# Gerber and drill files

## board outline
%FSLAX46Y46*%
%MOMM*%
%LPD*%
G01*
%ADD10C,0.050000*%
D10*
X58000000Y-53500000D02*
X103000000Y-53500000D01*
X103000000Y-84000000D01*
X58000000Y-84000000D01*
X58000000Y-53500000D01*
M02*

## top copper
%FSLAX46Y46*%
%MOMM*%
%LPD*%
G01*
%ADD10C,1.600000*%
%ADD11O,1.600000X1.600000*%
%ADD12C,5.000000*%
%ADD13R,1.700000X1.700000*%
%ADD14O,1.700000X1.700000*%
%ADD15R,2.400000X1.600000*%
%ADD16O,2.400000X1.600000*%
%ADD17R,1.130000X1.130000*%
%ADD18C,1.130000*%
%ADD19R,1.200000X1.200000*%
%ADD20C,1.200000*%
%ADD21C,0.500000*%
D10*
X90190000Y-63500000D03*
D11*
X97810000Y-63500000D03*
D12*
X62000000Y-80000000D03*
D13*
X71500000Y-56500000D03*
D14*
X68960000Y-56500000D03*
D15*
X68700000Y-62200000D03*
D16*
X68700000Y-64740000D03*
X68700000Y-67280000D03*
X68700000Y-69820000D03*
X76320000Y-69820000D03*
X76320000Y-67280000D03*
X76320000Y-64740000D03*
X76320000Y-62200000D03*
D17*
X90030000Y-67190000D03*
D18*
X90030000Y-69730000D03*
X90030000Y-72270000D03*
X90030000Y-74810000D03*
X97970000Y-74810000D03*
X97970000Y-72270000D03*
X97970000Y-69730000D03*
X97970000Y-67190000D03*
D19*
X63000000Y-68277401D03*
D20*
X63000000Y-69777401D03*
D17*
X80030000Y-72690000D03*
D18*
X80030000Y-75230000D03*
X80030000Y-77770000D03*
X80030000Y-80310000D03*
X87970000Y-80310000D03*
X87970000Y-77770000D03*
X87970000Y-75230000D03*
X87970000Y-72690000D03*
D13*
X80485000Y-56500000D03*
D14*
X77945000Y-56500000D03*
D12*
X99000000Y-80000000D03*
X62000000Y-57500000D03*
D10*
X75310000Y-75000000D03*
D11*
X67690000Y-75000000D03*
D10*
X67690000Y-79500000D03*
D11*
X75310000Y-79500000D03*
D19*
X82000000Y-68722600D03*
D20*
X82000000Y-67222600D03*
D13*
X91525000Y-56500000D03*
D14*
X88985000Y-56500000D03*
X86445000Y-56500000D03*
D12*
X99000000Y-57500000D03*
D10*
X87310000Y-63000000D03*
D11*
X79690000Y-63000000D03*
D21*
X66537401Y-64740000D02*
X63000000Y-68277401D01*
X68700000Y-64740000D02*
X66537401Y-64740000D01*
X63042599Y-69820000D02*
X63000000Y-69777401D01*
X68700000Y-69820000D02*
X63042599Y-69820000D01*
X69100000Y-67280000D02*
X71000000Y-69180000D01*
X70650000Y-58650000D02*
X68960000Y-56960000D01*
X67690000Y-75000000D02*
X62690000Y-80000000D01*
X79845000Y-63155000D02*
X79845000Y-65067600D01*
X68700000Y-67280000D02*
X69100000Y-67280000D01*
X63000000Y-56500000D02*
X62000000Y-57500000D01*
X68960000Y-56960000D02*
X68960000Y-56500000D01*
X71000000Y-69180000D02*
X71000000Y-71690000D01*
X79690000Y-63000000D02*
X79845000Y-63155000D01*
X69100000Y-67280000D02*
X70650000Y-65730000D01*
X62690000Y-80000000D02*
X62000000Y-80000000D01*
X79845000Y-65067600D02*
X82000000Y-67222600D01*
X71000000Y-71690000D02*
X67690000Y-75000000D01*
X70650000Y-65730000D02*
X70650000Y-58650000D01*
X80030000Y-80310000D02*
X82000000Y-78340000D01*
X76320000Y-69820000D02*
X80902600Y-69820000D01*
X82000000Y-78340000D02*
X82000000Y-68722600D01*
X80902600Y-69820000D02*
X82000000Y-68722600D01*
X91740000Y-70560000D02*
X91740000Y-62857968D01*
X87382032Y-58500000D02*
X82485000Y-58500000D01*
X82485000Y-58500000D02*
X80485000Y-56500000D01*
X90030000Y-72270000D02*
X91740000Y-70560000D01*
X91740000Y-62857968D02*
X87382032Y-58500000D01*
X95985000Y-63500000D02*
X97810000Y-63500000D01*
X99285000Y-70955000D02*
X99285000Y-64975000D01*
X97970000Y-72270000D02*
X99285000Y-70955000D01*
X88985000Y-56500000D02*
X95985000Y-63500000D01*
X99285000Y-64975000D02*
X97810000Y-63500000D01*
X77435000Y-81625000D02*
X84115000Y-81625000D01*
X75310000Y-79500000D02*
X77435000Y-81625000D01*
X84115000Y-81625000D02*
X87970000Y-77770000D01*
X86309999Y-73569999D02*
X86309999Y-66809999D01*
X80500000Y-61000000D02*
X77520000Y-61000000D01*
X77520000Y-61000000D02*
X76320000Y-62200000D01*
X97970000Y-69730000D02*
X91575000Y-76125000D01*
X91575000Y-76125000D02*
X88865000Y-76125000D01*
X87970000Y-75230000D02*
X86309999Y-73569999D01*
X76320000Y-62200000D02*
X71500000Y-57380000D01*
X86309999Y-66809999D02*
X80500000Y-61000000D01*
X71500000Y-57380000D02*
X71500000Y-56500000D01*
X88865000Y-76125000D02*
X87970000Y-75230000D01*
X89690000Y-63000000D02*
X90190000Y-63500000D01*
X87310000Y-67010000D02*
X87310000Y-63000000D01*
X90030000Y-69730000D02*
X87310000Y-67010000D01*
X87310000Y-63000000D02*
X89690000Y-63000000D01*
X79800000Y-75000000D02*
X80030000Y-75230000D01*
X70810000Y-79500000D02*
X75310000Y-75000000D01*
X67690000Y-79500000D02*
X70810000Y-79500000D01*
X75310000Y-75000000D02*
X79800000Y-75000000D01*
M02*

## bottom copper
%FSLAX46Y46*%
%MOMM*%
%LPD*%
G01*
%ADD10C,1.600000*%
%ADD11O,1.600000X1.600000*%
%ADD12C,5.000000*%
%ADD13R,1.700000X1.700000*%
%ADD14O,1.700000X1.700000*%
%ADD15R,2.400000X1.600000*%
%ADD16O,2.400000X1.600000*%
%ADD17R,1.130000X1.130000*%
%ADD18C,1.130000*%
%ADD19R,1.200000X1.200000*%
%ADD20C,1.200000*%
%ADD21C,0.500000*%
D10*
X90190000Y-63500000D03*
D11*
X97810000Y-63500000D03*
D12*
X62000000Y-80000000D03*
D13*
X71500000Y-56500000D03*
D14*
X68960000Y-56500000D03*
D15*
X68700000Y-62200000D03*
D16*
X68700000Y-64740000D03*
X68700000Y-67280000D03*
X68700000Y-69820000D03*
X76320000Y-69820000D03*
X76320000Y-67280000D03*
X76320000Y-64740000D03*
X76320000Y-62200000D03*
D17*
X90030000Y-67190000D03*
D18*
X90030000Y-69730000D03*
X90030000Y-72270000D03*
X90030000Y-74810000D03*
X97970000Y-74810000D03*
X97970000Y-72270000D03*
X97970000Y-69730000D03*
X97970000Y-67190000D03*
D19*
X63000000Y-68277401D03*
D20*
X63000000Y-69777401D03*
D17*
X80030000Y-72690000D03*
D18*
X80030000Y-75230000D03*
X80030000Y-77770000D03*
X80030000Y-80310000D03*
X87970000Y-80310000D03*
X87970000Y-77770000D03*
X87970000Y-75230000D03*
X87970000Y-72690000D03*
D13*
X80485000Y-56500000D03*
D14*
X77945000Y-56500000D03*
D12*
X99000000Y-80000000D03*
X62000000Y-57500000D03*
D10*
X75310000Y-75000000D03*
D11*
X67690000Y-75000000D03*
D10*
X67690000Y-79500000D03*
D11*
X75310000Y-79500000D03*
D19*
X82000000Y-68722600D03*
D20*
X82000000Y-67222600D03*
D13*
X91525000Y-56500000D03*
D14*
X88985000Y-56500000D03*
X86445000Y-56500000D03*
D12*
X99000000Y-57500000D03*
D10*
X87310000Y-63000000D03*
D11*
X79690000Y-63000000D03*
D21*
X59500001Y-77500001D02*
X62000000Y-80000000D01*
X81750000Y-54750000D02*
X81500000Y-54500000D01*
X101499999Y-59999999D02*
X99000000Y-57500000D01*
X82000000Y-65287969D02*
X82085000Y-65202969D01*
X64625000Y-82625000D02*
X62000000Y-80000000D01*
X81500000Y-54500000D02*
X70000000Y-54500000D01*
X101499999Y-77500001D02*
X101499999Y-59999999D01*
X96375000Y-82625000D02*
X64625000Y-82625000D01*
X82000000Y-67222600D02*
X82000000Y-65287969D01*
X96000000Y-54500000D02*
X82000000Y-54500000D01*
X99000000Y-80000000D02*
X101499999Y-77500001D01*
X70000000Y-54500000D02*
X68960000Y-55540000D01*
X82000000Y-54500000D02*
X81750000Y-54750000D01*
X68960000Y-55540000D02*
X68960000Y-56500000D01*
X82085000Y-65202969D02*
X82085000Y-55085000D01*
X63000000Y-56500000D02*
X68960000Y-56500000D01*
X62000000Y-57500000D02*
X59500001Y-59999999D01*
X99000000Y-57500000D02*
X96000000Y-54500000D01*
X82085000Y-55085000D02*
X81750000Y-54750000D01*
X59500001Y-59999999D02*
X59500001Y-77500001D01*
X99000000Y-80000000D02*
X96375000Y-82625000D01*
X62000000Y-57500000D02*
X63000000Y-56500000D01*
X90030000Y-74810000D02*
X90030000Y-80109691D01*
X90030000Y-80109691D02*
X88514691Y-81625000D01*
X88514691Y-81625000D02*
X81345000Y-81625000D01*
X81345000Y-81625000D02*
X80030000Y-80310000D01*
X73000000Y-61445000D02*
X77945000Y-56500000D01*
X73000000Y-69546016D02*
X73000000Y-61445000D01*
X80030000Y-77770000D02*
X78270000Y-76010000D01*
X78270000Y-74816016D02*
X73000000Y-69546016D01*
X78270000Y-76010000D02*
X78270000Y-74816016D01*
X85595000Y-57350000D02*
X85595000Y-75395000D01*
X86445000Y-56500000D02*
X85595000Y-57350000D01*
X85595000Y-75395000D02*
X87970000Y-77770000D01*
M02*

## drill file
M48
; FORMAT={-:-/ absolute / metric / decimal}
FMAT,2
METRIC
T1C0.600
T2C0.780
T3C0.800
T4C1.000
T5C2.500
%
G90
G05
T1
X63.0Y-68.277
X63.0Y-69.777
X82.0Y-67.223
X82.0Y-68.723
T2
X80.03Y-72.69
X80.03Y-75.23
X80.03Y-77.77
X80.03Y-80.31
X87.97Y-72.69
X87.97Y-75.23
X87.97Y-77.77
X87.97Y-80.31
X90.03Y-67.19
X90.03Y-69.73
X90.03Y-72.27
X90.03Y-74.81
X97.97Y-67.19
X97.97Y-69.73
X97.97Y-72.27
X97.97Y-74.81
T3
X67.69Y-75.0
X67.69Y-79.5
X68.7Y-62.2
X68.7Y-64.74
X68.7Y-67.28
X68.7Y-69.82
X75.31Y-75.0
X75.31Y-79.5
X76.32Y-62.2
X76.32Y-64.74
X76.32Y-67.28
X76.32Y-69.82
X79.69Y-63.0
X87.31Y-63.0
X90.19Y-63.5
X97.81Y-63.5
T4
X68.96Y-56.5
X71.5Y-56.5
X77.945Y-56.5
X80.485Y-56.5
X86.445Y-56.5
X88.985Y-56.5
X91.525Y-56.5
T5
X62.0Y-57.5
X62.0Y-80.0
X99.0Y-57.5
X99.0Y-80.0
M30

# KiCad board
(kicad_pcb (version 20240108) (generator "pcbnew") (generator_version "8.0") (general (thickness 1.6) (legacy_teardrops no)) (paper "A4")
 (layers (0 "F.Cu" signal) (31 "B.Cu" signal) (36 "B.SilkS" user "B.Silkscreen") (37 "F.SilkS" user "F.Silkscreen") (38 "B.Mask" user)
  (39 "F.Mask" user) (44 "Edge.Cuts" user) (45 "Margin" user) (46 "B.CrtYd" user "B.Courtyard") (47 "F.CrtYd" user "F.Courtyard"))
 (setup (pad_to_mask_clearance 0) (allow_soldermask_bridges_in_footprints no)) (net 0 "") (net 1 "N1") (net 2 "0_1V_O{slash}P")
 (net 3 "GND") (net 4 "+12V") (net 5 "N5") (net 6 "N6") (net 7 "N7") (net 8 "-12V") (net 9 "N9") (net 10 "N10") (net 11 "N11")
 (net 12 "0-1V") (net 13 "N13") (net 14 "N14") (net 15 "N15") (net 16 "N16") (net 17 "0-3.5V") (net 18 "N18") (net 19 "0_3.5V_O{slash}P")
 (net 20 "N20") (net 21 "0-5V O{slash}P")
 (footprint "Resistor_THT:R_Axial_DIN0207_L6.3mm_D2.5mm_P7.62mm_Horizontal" (layer "F.Cu") (at 90.19 63.5)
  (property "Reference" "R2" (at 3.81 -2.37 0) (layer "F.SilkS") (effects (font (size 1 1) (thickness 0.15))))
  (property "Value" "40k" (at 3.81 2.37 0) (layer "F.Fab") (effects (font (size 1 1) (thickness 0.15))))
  (pad "1" thru_hole circle (at 0 0) (size 1.6 1.6) (drill 0.8) (layers "*.Cu" "*.Mask") (remove_unused_layers no) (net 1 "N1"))
  (pad "2" thru_hole oval (at 7.62 0) (size 1.6 1.6) (drill 0.8) (layers "*.Cu" "*.Mask") (remove_unused_layers no) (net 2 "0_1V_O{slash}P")))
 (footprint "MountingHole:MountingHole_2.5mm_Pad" (layer "F.Cu") (at 62 80 180)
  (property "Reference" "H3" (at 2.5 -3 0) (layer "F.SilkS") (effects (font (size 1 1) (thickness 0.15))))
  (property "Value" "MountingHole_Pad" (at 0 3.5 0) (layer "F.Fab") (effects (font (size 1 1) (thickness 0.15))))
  (pad "1" thru_hole circle (at 0 0 180) (size 5 5) (drill 2.5) (layers "*.Cu" "*.Mask") (remove_unused_layers no) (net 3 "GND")))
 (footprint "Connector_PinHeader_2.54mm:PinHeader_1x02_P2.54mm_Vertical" (layer "F.Cu") (at 71.5 56.5 -90)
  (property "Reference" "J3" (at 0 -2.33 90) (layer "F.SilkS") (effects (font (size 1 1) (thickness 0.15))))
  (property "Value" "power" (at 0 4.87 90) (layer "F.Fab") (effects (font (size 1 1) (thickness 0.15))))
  (pad "1" thru_hole rect (at 0 0 270) (size 1.7 1.7) (drill 1) (layers "*.Cu" "*.Mask") (remove_unused_layers no) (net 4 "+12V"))
  (pad "2" thru_hole oval (at 0 2.54 270) (size 1.7 1.7) (drill 1) (layers "*.Cu" "*.Mask") (remove_unused_layers no) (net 3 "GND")))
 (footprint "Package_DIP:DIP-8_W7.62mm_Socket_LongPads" (layer "F.Cu") (at 68.7 62.2)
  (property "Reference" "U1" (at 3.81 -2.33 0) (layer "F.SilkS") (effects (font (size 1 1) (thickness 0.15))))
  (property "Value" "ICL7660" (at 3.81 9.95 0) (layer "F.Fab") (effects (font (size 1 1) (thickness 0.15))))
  (pad "1" thru_hole rect (at 0 0) (size 2.4 1.6) (drill 0.8) (layers "*.Cu" "*.Mask") (remove_unused_layers no) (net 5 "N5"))
  (pad "2" thru_hole oval (at 0 2.54) (size 2.4 1.6) (drill 0.8) (layers "*.Cu" "*.Mask") (remove_unused_layers no) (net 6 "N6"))
  (pad "3" thru_hole oval (at 0 5.08) (size 2.4 1.6) (drill 0.8) (layers "*.Cu" "*.Mask") (remove_unused_layers no) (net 3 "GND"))
  (pad "4" thru_hole oval (at 0 7.62) (size 2.4 1.6) (drill 0.8) (layers "*.Cu" "*.Mask") (remove_unused_layers no) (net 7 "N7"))
  (pad "5" thru_hole oval (at 7.62 7.62) (size 2.4 1.6) (drill 0.8) (layers "*.Cu" "*.Mask") (remove_unused_layers no) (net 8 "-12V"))
  (pad "6" thru_hole oval (at 7.62 5.08) (size 2.4 1.6) (drill 0.8) (layers "*.Cu" "*.Mask") (remove_unused_layers no) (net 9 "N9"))
  (pad "7" thru_hole oval (at 7.62 2.54) (size 2.4 1.6) (drill 0.8) (layers "*.Cu" "*.Mask") (remove_unused_layers no) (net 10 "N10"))
  (pad "8" thru_hole oval (at 7.62 0) (size 2.4 1.6) (drill 0.8) (layers "*.Cu" "*.Mask") (remove_unused_layers no) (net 4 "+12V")))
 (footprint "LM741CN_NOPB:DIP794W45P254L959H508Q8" (layer "F.Cu") (at 94 71)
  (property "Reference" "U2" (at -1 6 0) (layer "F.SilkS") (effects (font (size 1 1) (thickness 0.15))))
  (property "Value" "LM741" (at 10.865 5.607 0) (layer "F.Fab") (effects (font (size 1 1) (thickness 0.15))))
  (pad "1" thru_hole rect (at -3.97 -3.81) (size 1.13 1.13) (drill 0.78) (layers "*.Cu" "*.Mask") (remove_unused_layers no) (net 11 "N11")
   (solder_mask_margin 0.102))
  (pad "2" thru_hole circle (at -3.97 -1.27) (size 1.13 1.13) (drill 0.78) (layers "*.Cu" "*.Mask") (remove_unused_layers no) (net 1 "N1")
   (solder_mask_margin 0.102))
  (pad "3" thru_hole circle (at -3.97 1.27) (size 1.13 1.13) (drill 0.78) (layers "*.Cu" "*.Mask") (remove_unused_layers no) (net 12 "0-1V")
   (solder_mask_margin 0.102))
  (pad "4" thru_hole circle (at -3.97 3.81) (size 1.13 1.13) (drill 0.78) (layers "*.Cu" "*.Mask") (remove_unused_layers no) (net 8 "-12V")
   (solder_mask_margin 0.102))
  (pad "5" thru_hole circle (at 3.97 3.81) (size 1.13 1.13) (drill 0.78) (layers "*.Cu" "*.Mask") (remove_unused_layers no) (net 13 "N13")
   (solder_mask_margin 0.102))
  (pad "6" thru_hole circle (at 3.97 1.27) (size 1.13 1.13) (drill 0.78) (layers "*.Cu" "*.Mask") (remove_unused_layers no)
   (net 2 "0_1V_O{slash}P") (solder_mask_margin 0.102))
  (pad "7" thru_hole circle (at 3.97 -1.27) (size 1.13 1.13) (drill 0.78) (layers "*.Cu" "*.Mask") (remove_unused_layers no) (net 4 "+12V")
   (solder_mask_margin 0.102))
  (pad "8" thru_hole circle (at 3.97 -3.81) (size 1.13 1.13) (drill 0.78) (layers "*.Cu" "*.Mask") (remove_unused_layers no) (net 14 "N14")
   (solder_mask_margin 0.102)))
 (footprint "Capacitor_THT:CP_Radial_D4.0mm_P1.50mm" (layer "F.Cu") (at 63 68.277401 -90)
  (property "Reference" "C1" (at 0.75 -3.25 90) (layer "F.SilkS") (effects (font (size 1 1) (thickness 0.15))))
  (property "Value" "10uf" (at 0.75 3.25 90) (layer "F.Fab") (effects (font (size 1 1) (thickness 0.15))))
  (pad "1" thru_hole rect (at 0 0 270) (size 1.2 1.2) (drill 0.6) (layers "*.Cu" "*.Mask") (remove_unused_layers no) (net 6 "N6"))
  (pad "2" thru_hole circle (at 1.5 0 270) (size 1.2 1.2) (drill 0.6) (layers "*.Cu" "*.Mask") (remove_unused_layers no) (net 7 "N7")))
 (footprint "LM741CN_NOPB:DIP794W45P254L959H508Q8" (layer "F.Cu") (at 84 76.5)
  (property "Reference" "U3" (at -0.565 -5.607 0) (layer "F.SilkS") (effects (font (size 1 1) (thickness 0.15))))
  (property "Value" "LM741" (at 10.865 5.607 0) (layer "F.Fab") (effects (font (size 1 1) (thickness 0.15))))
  (pad "1" thru_hole rect (at -3.97 -3.81) (size 1.13 1.13) (drill 0.78) (layers "*.Cu" "*.Mask") (remove_unused_layers no) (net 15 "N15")
   (solder_mask_margin 0.102))
  (pad "2" thru_hole circle (at -3.97 -1.27) (size 1.13 1.13) (drill 0.78) (layers "*.Cu" "*.Mask") (remove_unused_layers no) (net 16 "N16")
   (solder_mask_margin 0.102))
  (pad "3" thru_hole circle (at -3.97 1.27) (size 1.13 1.13) (drill 0.78) (layers "*.Cu" "*.Mask") (remove_unused_layers no)
   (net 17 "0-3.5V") (solder_mask_margin 0.102))
  (pad "4" thru_hole circle (at -3.97 3.81) (size 1.13 1.13) (drill 0.78) (layers "*.Cu" "*.Mask") (remove_unused_layers no) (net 8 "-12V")
   (solder_mask_margin 0.102))
  (pad "5" thru_hole circle (at 3.97 3.81) (size 1.13 1.13) (drill 0.78) (layers "*.Cu" "*.Mask") (remove_unused_layers no) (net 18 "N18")
   (solder_mask_margin 0.102))
  (pad "6" thru_hole circle (at 3.97 1.27) (size 1.13 1.13) (drill 0.78) (layers "*.Cu" "*.Mask") (remove_unused_layers no)
   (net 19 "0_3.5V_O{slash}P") (solder_mask_margin 0.102))
  (pad "7" thru_hole circle (at 3.97 -1.27) (size 1.13 1.13) (drill 0.78) (layers "*.Cu" "*.Mask") (remove_unused_layers no) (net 4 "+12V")
   (solder_mask_margin 0.102))
  (pad "8" thru_hole circle (at 3.97 -3.81) (size 1.13 1.13) (drill 0.78) (layers "*.Cu" "*.Mask") (remove_unused_layers no) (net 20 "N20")
   (solder_mask_margin 0.102)))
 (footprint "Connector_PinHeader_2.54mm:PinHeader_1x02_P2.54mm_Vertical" (layer "F.Cu") (at 80.485 56.5 -90)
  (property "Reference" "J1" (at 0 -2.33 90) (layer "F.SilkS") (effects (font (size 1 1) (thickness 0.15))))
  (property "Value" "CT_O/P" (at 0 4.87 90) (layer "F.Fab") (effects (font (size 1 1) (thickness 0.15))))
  (pad "1" thru_hole rect (at 0 0 270) (size 1.7 1.7) (drill 1) (layers "*.Cu" "*.Mask") (remove_unused_layers no) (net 12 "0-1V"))
  (pad "2" thru_hole oval (at 0 2.54 270) (size 1.7 1.7) (drill 1) (layers "*.Cu" "*.Mask") (remove_unused_layers no) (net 17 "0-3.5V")))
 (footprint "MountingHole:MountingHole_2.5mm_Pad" (layer "F.Cu") (at 99 80 180)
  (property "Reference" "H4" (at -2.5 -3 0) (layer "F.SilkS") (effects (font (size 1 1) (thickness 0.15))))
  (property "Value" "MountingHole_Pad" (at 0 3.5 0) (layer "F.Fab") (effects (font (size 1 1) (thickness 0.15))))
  (pad "1" thru_hole circle (at 0 0 180) (size 5 5) (drill 2.5) (layers "*.Cu" "*.Mask") (remove_unused_layers no) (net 3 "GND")))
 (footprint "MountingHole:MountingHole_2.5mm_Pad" (layer "F.Cu") (at 62 57.5 180)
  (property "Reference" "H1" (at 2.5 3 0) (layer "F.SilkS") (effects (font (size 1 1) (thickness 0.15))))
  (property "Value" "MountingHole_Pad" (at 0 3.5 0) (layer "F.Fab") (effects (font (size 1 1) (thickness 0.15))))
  (pad "1" thru_hole circle (at 0 0 180) (size 5 5) (drill 2.5) (layers "*.Cu" "*.Mask") (remove_unused_layers no) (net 3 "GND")))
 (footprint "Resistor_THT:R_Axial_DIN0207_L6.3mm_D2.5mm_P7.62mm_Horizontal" (layer "F.Cu") (at 75.31 75 180)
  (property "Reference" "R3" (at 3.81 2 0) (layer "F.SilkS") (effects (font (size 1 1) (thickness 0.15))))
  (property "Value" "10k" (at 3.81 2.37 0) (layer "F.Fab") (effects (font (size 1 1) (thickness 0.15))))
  (pad "1" thru_hole circle (at 0 0 180) (size 1.6 1.6) (drill 0.8) (layers "*.Cu" "*.Mask") (remove_unused_layers no) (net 16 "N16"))
  (pad "2" thru_hole oval (at 7.62 0 180) (size 1.6 1.6) (drill 0.8) (layers "*.Cu" "*.Mask") (remove_unused_layers no) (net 3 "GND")))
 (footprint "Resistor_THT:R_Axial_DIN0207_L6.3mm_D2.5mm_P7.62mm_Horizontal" (layer "F.Cu") (at 67.69 79.5)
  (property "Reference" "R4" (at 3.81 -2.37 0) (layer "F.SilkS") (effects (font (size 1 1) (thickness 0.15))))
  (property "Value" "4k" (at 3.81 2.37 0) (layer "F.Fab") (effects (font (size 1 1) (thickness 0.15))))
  (pad "1" thru_hole circle (at 0 0) (size 1.6 1.6) (drill 0.8) (layers "*.Cu" "*.Mask") (remove_unused_layers no) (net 16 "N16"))
  (pad "2" thru_hole oval (at 7.62 0) (size 1.6 1.6) (drill 0.8) (layers "*.Cu" "*.Mask") (remove_unused_layers no)
   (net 19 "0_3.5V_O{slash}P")))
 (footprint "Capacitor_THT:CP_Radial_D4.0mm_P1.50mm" (layer "F.Cu") (at 82 68.7226 90)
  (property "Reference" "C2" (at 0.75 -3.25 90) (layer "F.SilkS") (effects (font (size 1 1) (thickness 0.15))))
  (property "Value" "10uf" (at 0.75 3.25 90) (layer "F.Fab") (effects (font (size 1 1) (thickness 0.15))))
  (pad "1" thru_hole rect (at 0 0 90) (size 1.2 1.2) (drill 0.6) (layers "*.Cu" "*.Mask") (remove_unused_layers no) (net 8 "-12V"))
  (pad "2" thru_hole circle (at 1.5 0 90) (size 1.2 1.2) (drill 0.6) (layers "*.Cu" "*.Mask") (remove_unused_layers no) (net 3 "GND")))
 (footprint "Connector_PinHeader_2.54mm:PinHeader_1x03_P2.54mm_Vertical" (layer "F.Cu") (at 91.525 56.5 -90)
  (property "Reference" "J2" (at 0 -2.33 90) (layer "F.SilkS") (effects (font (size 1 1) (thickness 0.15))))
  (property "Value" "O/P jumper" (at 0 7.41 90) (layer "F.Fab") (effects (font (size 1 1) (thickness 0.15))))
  (pad "1" thru_hole rect (at 0 0 270) (size 1.7 1.7) (drill 1) (layers "*.Cu" "*.Mask") (remove_unused_layers no) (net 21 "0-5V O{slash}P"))
  (pad "2" thru_hole oval (at 0 2.54 270) (size 1.7 1.7) (drill 1) (layers "*.Cu" "*.Mask") (remove_unused_layers no)
   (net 2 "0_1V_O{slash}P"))
  (pad "3" thru_hole oval (at 0 5.08 270) (size 1.7 1.7) (drill 1) (layers "*.Cu" "*.Mask") (remove_unused_layers no)
   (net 19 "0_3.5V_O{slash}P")))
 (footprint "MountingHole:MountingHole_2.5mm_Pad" (layer "F.Cu") (at 99 57.5 180)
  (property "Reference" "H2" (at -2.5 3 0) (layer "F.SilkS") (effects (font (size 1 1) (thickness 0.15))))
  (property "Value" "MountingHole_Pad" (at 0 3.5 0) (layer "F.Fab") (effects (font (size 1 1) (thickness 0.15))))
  (pad "1" thru_hole circle (at 0 0 180) (size 5 5) (drill 2.5) (layers "*.Cu" "*.Mask") (remove_unused_layers no) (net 3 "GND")))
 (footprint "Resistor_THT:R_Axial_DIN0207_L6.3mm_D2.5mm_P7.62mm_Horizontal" (layer "F.Cu") (at 87.31 63 180)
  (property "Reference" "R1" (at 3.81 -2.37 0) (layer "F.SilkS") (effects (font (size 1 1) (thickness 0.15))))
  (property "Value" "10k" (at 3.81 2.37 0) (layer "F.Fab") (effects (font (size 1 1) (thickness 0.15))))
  (pad "1" thru_hole circle (at 0 0 180) (size 1.6 1.6) (drill 0.8) (layers "*.Cu" "*.Mask") (remove_unused_layers no) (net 1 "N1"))
  (pad "2" thru_hole oval (at 7.62 0 180) (size 1.6 1.6) (drill 0.8) (layers "*.Cu" "*.Mask") (remove_unused_layers no) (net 3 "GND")))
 (gr_rect (start 58 53.5) (end 103 84) (stroke (width 0.05) (type default)) (fill none) (layer "Edge.Cuts"))
 (segment (start 66.537401 64.74) (end 63 68.277401) (width 0.5) (layer "F.Cu") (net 6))
 (segment (start 68.7 64.74) (end 66.537401 64.74) (width 0.5) (layer "F.Cu") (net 6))
 (segment (start 63.042599 69.82) (end 63 69.777401) (width 0.5) (layer "F.Cu") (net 7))
 (segment (start 68.7 69.82) (end 63.042599 69.82) (width 0.5) (layer "F.Cu") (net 7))
 (segment (start 69.1 67.28) (end 71 69.18) (width 0.5) (layer "F.Cu") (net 3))
 (segment (start 70.65 58.65) (end 68.96 56.96) (width 0.5) (layer "F.Cu") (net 3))
 (segment (start 67.69 75) (end 62.69 80) (width 0.5) (layer "F.Cu") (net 3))
 (segment (start 79.845 63.155) (end 79.845 65.0676) (width 0.5) (layer "F.Cu") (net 3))
 (segment (start 68.7 67.28) (end 69.1 67.28) (width 0.5) (layer "F.Cu") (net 3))
 (segment (start 63 56.5) (end 62 57.5) (width 0.5) (layer "F.Cu") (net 3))
 (segment (start 68.96 56.96) (end 68.96 56.5) (width 0.5) (layer "F.Cu") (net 3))
 (segment (start 71 69.18) (end 71 71.69) (width 0.5) (layer "F.Cu") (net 3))
 (segment (start 79.69 63) (end 79.845 63.155) (width 0.5) (layer "F.Cu") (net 3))
 (segment (start 69.1 67.28) (end 70.65 65.73) (width 0.5) (layer "F.Cu") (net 3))
 (segment (start 62.69 80) (end 62 80) (width 0.5) (layer "F.Cu") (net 3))
 (segment (start 79.845 65.0676) (end 82 67.2226) (width 0.5) (layer "F.Cu") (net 3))
 (segment (start 71 71.69) (end 67.69 75) (width 0.5) (layer "F.Cu") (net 3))
 (segment (start 70.65 65.73) (end 70.65 58.65) (width 0.5) (layer "F.Cu") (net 3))
 (segment (start 59.500001 77.500001) (end 62 80) (width 0.5) (layer "B.Cu") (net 3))
 (segment (start 81.75 54.75) (end 81.5 54.5) (width 0.5) (layer "B.Cu") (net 3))
 (segment (start 101.499999 59.999999) (end 99 57.5) (width 0.5) (layer "B.Cu") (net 3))
 (segment (start 82 65.287969) (end 82.085 65.202969) (width 0.5) (layer "B.Cu") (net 3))
 (segment (start 64.625 82.625) (end 62 80) (width 0.5) (layer "B.Cu") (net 3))
 (segment (start 81.5 54.5) (end 70 54.5) (width 0.5) (layer "B.Cu") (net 3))
 (segment (start 101.499999 77.500001) (end 101.499999 59.999999) (width 0.5) (layer "B.Cu") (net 3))
 (segment (start 96.375 82.625) (end 64.625 82.625) (width 0.5) (layer "B.Cu") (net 3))
 (segment (start 82 67.2226) (end 82 65.287969) (width 0.5) (layer "B.Cu") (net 3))
 (segment (start 96 54.5) (end 82 54.5) (width 0.5) (layer "B.Cu") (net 3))
 (segment (start 99 80) (end 101.499999 77.500001) (width 0.5) (layer "B.Cu") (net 3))
 (segment (start 70 54.5) (end 68.96 55.54) (width 0.5) (layer "B.Cu") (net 3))
 (segment (start 82 54.5) (end 81.75 54.75) (width 0.5) (layer "B.Cu") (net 3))
 (segment (start 68.96 55.54) (end 68.96 56.5) (width 0.5) (layer "B.Cu") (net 3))
 (segment (start 82.085 65.202969) (end 82.085 55.085) (width 0.5) (layer "B.Cu") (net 3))
 (segment (start 63 56.5) (end 68.96 56.5) (width 0.5) (layer "B.Cu") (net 3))
 (segment (start 62 57.5) (end 59.500001 59.999999) (width 0.5) (layer "B.Cu") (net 3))
 (segment (start 99 57.5) (end 96 54.5) (width 0.5) (layer "B.Cu") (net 3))
 (segment (start 82.085 55.085) (end 81.75 54.75) (width 0.5) (layer "B.Cu") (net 3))
 (segment (start 59.500001 59.999999) (end 59.500001 77.500001) (width 0.5) (layer "B.Cu") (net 3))
 (segment (start 99 80) (end 96.375 82.625) (width 0.5) (layer "B.Cu") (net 3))
 (segment (start 62 57.5) (end 63 56.5) (width 0.5) (layer "B.Cu") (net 3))
 (segment (start 80.03 80.31) (end 82 78.34) (width 0.5) (layer "F.Cu") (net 8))
 (segment (start 76.32 69.82) (end 80.9026 69.82) (width 0.5) (layer "F.Cu") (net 8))
 (segment (start 82 78.34) (end 82 68.7226) (width 0.5) (layer "F.Cu") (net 8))
 (segment (start 80.9026 69.82) (end 82 68.7226) (width 0.5) (layer "F.Cu") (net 8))
 (segment (start 90.03 74.81) (end 90.03 80.109691) (width 0.5) (layer "B.Cu") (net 8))
 (segment (start 90.03 80.109691) (end 88.514691 81.625) (width 0.5) (layer "B.Cu") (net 8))
 (segment (start 88.514691 81.625) (end 81.345 81.625) (width 0.5) (layer "B.Cu") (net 8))
 (segment (start 81.345 81.625) (end 80.03 80.31) (width 0.5) (layer "B.Cu") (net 8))
 (segment (start 91.74 70.56) (end 91.74 62.857968) (width 0.5) (layer "F.Cu") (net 12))
 (segment (start 87.382032 58.5) (end 82.485 58.5) (width 0.5) (layer "F.Cu") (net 12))
 (segment (start 82.485 58.5) (end 80.485 56.5) (width 0.5) (layer "F.Cu") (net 12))
 (segment (start 90.03 72.27) (end 91.74 70.56) (width 0.5) (layer "F.Cu") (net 12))
 (segment (start 91.74 62.857968) (end 87.382032 58.5) (width 0.5) (layer "F.Cu") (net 12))
 (segment (start 73 61.445) (end 77.945 56.5) (width 0.5) (layer "B.Cu") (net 17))
 (segment (start 73 69.546016) (end 73 61.445) (width 0.5) (layer "B.Cu") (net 17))
 (segment (start 80.03 77.77) (end 78.27 76.01) (width 0.5) (layer "B.Cu") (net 17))
 (segment (start 78.27 74.816016) (end 73 69.546016) (width 0.5) (layer "B.Cu") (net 17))
 (segment (start 78.27 76.01) (end 78.27 74.816016) (width 0.5) (layer "B.Cu") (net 17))
 (segment (start 95.985 63.5) (end 97.81 63.5) (width 0.5) (layer "F.Cu") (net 2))
 (segment (start 99.285 70.955) (end 99.285 64.975) (width 0.5) (layer "F.Cu") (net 2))
 (segment (start 97.97 72.27) (end 99.285 70.955) (width 0.5) (layer "F.Cu") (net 2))
 (segment (start 88.985 56.5) (end 95.985 63.5) (width 0.5) (layer "F.Cu") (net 2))
 (segment (start 99.285 64.975) (end 97.81 63.5) (width 0.5) (layer "F.Cu") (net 2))
 (segment (start 77.435 81.625) (end 84.115 81.625) (width 0.5) (layer "F.Cu") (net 19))
 (segment (start 75.31 79.5) (end 77.435 81.625) (width 0.5) (layer "F.Cu") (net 19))
 (segment (start 84.115 81.625) (end 87.97 77.77) (width 0.5) (layer "F.Cu") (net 19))
 (segment (start 85.595 57.35) (end 85.595 75.395) (width 0.5) (layer "B.Cu") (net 19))
 (segment (start 86.445 56.5) (end 85.595 57.35) (width 0.5) (layer "B.Cu") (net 19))
 (segment (start 85.595 75.395) (end 87.97 77.77) (width 0.5) (layer "B.Cu") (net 19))
 (segment (start 86.309999 73.569999) (end 86.309999 66.809999) (width 0.5) (layer "F.Cu") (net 4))
 (segment (start 80.5 61) (end 77.52 61) (width 0.5) (layer "F.Cu") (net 4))
 (segment (start 77.52 61) (end 76.32 62.2) (width 0.5) (layer "F.Cu") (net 4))
 (segment (start 97.97 69.73) (end 91.575 76.125) (width 0.5) (layer "F.Cu") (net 4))
 (segment (start 91.575 76.125) (end 88.865 76.125) (width 0.5) (layer "F.Cu") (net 4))
 (segment (start 87.97 75.23) (end 86.309999 73.569999) (width 0.5) (layer "F.Cu") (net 4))
 (segment (start 76.32 62.2) (end 71.5 57.38) (width 0.5) (layer "F.Cu") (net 4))
 (segment (start 86.309999 66.809999) (end 80.5 61) (width 0.5) (layer "F.Cu") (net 4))
 (segment (start 71.5 57.38) (end 71.5 56.5) (width 0.5) (layer "F.Cu") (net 4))
 (segment (start 88.865 76.125) (end 87.97 75.23) (width 0.5) (layer "F.Cu") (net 4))
 (segment (start 89.69 63) (end 90.19 63.5) (width 0.5) (layer "F.Cu") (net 1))
 (segment (start 87.31 67.01) (end 87.31 63) (width 0.5) (layer "F.Cu") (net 1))
 (segment (start 90.03 69.73) (end 87.31 67.01) (width 0.5) (layer "F.Cu") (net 1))
 (segment (start 87.31 63) (end 89.69 63) (width 0.5) (layer "F.Cu") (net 1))
 (segment (start 79.8 75) (end 80.03 75.23) (width 0.5) (layer "F.Cu") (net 16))
 (segment (start 70.81 79.5) (end 75.31 75) (width 0.5) (layer "F.Cu") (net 16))
 (segment (start 67.69 79.5) (end 70.81 79.5) (width 0.5) (layer "F.Cu") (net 16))
 (segment (start 75.31 75) (end 79.8 75) (width 0.5) (layer "F.Cu") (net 16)))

